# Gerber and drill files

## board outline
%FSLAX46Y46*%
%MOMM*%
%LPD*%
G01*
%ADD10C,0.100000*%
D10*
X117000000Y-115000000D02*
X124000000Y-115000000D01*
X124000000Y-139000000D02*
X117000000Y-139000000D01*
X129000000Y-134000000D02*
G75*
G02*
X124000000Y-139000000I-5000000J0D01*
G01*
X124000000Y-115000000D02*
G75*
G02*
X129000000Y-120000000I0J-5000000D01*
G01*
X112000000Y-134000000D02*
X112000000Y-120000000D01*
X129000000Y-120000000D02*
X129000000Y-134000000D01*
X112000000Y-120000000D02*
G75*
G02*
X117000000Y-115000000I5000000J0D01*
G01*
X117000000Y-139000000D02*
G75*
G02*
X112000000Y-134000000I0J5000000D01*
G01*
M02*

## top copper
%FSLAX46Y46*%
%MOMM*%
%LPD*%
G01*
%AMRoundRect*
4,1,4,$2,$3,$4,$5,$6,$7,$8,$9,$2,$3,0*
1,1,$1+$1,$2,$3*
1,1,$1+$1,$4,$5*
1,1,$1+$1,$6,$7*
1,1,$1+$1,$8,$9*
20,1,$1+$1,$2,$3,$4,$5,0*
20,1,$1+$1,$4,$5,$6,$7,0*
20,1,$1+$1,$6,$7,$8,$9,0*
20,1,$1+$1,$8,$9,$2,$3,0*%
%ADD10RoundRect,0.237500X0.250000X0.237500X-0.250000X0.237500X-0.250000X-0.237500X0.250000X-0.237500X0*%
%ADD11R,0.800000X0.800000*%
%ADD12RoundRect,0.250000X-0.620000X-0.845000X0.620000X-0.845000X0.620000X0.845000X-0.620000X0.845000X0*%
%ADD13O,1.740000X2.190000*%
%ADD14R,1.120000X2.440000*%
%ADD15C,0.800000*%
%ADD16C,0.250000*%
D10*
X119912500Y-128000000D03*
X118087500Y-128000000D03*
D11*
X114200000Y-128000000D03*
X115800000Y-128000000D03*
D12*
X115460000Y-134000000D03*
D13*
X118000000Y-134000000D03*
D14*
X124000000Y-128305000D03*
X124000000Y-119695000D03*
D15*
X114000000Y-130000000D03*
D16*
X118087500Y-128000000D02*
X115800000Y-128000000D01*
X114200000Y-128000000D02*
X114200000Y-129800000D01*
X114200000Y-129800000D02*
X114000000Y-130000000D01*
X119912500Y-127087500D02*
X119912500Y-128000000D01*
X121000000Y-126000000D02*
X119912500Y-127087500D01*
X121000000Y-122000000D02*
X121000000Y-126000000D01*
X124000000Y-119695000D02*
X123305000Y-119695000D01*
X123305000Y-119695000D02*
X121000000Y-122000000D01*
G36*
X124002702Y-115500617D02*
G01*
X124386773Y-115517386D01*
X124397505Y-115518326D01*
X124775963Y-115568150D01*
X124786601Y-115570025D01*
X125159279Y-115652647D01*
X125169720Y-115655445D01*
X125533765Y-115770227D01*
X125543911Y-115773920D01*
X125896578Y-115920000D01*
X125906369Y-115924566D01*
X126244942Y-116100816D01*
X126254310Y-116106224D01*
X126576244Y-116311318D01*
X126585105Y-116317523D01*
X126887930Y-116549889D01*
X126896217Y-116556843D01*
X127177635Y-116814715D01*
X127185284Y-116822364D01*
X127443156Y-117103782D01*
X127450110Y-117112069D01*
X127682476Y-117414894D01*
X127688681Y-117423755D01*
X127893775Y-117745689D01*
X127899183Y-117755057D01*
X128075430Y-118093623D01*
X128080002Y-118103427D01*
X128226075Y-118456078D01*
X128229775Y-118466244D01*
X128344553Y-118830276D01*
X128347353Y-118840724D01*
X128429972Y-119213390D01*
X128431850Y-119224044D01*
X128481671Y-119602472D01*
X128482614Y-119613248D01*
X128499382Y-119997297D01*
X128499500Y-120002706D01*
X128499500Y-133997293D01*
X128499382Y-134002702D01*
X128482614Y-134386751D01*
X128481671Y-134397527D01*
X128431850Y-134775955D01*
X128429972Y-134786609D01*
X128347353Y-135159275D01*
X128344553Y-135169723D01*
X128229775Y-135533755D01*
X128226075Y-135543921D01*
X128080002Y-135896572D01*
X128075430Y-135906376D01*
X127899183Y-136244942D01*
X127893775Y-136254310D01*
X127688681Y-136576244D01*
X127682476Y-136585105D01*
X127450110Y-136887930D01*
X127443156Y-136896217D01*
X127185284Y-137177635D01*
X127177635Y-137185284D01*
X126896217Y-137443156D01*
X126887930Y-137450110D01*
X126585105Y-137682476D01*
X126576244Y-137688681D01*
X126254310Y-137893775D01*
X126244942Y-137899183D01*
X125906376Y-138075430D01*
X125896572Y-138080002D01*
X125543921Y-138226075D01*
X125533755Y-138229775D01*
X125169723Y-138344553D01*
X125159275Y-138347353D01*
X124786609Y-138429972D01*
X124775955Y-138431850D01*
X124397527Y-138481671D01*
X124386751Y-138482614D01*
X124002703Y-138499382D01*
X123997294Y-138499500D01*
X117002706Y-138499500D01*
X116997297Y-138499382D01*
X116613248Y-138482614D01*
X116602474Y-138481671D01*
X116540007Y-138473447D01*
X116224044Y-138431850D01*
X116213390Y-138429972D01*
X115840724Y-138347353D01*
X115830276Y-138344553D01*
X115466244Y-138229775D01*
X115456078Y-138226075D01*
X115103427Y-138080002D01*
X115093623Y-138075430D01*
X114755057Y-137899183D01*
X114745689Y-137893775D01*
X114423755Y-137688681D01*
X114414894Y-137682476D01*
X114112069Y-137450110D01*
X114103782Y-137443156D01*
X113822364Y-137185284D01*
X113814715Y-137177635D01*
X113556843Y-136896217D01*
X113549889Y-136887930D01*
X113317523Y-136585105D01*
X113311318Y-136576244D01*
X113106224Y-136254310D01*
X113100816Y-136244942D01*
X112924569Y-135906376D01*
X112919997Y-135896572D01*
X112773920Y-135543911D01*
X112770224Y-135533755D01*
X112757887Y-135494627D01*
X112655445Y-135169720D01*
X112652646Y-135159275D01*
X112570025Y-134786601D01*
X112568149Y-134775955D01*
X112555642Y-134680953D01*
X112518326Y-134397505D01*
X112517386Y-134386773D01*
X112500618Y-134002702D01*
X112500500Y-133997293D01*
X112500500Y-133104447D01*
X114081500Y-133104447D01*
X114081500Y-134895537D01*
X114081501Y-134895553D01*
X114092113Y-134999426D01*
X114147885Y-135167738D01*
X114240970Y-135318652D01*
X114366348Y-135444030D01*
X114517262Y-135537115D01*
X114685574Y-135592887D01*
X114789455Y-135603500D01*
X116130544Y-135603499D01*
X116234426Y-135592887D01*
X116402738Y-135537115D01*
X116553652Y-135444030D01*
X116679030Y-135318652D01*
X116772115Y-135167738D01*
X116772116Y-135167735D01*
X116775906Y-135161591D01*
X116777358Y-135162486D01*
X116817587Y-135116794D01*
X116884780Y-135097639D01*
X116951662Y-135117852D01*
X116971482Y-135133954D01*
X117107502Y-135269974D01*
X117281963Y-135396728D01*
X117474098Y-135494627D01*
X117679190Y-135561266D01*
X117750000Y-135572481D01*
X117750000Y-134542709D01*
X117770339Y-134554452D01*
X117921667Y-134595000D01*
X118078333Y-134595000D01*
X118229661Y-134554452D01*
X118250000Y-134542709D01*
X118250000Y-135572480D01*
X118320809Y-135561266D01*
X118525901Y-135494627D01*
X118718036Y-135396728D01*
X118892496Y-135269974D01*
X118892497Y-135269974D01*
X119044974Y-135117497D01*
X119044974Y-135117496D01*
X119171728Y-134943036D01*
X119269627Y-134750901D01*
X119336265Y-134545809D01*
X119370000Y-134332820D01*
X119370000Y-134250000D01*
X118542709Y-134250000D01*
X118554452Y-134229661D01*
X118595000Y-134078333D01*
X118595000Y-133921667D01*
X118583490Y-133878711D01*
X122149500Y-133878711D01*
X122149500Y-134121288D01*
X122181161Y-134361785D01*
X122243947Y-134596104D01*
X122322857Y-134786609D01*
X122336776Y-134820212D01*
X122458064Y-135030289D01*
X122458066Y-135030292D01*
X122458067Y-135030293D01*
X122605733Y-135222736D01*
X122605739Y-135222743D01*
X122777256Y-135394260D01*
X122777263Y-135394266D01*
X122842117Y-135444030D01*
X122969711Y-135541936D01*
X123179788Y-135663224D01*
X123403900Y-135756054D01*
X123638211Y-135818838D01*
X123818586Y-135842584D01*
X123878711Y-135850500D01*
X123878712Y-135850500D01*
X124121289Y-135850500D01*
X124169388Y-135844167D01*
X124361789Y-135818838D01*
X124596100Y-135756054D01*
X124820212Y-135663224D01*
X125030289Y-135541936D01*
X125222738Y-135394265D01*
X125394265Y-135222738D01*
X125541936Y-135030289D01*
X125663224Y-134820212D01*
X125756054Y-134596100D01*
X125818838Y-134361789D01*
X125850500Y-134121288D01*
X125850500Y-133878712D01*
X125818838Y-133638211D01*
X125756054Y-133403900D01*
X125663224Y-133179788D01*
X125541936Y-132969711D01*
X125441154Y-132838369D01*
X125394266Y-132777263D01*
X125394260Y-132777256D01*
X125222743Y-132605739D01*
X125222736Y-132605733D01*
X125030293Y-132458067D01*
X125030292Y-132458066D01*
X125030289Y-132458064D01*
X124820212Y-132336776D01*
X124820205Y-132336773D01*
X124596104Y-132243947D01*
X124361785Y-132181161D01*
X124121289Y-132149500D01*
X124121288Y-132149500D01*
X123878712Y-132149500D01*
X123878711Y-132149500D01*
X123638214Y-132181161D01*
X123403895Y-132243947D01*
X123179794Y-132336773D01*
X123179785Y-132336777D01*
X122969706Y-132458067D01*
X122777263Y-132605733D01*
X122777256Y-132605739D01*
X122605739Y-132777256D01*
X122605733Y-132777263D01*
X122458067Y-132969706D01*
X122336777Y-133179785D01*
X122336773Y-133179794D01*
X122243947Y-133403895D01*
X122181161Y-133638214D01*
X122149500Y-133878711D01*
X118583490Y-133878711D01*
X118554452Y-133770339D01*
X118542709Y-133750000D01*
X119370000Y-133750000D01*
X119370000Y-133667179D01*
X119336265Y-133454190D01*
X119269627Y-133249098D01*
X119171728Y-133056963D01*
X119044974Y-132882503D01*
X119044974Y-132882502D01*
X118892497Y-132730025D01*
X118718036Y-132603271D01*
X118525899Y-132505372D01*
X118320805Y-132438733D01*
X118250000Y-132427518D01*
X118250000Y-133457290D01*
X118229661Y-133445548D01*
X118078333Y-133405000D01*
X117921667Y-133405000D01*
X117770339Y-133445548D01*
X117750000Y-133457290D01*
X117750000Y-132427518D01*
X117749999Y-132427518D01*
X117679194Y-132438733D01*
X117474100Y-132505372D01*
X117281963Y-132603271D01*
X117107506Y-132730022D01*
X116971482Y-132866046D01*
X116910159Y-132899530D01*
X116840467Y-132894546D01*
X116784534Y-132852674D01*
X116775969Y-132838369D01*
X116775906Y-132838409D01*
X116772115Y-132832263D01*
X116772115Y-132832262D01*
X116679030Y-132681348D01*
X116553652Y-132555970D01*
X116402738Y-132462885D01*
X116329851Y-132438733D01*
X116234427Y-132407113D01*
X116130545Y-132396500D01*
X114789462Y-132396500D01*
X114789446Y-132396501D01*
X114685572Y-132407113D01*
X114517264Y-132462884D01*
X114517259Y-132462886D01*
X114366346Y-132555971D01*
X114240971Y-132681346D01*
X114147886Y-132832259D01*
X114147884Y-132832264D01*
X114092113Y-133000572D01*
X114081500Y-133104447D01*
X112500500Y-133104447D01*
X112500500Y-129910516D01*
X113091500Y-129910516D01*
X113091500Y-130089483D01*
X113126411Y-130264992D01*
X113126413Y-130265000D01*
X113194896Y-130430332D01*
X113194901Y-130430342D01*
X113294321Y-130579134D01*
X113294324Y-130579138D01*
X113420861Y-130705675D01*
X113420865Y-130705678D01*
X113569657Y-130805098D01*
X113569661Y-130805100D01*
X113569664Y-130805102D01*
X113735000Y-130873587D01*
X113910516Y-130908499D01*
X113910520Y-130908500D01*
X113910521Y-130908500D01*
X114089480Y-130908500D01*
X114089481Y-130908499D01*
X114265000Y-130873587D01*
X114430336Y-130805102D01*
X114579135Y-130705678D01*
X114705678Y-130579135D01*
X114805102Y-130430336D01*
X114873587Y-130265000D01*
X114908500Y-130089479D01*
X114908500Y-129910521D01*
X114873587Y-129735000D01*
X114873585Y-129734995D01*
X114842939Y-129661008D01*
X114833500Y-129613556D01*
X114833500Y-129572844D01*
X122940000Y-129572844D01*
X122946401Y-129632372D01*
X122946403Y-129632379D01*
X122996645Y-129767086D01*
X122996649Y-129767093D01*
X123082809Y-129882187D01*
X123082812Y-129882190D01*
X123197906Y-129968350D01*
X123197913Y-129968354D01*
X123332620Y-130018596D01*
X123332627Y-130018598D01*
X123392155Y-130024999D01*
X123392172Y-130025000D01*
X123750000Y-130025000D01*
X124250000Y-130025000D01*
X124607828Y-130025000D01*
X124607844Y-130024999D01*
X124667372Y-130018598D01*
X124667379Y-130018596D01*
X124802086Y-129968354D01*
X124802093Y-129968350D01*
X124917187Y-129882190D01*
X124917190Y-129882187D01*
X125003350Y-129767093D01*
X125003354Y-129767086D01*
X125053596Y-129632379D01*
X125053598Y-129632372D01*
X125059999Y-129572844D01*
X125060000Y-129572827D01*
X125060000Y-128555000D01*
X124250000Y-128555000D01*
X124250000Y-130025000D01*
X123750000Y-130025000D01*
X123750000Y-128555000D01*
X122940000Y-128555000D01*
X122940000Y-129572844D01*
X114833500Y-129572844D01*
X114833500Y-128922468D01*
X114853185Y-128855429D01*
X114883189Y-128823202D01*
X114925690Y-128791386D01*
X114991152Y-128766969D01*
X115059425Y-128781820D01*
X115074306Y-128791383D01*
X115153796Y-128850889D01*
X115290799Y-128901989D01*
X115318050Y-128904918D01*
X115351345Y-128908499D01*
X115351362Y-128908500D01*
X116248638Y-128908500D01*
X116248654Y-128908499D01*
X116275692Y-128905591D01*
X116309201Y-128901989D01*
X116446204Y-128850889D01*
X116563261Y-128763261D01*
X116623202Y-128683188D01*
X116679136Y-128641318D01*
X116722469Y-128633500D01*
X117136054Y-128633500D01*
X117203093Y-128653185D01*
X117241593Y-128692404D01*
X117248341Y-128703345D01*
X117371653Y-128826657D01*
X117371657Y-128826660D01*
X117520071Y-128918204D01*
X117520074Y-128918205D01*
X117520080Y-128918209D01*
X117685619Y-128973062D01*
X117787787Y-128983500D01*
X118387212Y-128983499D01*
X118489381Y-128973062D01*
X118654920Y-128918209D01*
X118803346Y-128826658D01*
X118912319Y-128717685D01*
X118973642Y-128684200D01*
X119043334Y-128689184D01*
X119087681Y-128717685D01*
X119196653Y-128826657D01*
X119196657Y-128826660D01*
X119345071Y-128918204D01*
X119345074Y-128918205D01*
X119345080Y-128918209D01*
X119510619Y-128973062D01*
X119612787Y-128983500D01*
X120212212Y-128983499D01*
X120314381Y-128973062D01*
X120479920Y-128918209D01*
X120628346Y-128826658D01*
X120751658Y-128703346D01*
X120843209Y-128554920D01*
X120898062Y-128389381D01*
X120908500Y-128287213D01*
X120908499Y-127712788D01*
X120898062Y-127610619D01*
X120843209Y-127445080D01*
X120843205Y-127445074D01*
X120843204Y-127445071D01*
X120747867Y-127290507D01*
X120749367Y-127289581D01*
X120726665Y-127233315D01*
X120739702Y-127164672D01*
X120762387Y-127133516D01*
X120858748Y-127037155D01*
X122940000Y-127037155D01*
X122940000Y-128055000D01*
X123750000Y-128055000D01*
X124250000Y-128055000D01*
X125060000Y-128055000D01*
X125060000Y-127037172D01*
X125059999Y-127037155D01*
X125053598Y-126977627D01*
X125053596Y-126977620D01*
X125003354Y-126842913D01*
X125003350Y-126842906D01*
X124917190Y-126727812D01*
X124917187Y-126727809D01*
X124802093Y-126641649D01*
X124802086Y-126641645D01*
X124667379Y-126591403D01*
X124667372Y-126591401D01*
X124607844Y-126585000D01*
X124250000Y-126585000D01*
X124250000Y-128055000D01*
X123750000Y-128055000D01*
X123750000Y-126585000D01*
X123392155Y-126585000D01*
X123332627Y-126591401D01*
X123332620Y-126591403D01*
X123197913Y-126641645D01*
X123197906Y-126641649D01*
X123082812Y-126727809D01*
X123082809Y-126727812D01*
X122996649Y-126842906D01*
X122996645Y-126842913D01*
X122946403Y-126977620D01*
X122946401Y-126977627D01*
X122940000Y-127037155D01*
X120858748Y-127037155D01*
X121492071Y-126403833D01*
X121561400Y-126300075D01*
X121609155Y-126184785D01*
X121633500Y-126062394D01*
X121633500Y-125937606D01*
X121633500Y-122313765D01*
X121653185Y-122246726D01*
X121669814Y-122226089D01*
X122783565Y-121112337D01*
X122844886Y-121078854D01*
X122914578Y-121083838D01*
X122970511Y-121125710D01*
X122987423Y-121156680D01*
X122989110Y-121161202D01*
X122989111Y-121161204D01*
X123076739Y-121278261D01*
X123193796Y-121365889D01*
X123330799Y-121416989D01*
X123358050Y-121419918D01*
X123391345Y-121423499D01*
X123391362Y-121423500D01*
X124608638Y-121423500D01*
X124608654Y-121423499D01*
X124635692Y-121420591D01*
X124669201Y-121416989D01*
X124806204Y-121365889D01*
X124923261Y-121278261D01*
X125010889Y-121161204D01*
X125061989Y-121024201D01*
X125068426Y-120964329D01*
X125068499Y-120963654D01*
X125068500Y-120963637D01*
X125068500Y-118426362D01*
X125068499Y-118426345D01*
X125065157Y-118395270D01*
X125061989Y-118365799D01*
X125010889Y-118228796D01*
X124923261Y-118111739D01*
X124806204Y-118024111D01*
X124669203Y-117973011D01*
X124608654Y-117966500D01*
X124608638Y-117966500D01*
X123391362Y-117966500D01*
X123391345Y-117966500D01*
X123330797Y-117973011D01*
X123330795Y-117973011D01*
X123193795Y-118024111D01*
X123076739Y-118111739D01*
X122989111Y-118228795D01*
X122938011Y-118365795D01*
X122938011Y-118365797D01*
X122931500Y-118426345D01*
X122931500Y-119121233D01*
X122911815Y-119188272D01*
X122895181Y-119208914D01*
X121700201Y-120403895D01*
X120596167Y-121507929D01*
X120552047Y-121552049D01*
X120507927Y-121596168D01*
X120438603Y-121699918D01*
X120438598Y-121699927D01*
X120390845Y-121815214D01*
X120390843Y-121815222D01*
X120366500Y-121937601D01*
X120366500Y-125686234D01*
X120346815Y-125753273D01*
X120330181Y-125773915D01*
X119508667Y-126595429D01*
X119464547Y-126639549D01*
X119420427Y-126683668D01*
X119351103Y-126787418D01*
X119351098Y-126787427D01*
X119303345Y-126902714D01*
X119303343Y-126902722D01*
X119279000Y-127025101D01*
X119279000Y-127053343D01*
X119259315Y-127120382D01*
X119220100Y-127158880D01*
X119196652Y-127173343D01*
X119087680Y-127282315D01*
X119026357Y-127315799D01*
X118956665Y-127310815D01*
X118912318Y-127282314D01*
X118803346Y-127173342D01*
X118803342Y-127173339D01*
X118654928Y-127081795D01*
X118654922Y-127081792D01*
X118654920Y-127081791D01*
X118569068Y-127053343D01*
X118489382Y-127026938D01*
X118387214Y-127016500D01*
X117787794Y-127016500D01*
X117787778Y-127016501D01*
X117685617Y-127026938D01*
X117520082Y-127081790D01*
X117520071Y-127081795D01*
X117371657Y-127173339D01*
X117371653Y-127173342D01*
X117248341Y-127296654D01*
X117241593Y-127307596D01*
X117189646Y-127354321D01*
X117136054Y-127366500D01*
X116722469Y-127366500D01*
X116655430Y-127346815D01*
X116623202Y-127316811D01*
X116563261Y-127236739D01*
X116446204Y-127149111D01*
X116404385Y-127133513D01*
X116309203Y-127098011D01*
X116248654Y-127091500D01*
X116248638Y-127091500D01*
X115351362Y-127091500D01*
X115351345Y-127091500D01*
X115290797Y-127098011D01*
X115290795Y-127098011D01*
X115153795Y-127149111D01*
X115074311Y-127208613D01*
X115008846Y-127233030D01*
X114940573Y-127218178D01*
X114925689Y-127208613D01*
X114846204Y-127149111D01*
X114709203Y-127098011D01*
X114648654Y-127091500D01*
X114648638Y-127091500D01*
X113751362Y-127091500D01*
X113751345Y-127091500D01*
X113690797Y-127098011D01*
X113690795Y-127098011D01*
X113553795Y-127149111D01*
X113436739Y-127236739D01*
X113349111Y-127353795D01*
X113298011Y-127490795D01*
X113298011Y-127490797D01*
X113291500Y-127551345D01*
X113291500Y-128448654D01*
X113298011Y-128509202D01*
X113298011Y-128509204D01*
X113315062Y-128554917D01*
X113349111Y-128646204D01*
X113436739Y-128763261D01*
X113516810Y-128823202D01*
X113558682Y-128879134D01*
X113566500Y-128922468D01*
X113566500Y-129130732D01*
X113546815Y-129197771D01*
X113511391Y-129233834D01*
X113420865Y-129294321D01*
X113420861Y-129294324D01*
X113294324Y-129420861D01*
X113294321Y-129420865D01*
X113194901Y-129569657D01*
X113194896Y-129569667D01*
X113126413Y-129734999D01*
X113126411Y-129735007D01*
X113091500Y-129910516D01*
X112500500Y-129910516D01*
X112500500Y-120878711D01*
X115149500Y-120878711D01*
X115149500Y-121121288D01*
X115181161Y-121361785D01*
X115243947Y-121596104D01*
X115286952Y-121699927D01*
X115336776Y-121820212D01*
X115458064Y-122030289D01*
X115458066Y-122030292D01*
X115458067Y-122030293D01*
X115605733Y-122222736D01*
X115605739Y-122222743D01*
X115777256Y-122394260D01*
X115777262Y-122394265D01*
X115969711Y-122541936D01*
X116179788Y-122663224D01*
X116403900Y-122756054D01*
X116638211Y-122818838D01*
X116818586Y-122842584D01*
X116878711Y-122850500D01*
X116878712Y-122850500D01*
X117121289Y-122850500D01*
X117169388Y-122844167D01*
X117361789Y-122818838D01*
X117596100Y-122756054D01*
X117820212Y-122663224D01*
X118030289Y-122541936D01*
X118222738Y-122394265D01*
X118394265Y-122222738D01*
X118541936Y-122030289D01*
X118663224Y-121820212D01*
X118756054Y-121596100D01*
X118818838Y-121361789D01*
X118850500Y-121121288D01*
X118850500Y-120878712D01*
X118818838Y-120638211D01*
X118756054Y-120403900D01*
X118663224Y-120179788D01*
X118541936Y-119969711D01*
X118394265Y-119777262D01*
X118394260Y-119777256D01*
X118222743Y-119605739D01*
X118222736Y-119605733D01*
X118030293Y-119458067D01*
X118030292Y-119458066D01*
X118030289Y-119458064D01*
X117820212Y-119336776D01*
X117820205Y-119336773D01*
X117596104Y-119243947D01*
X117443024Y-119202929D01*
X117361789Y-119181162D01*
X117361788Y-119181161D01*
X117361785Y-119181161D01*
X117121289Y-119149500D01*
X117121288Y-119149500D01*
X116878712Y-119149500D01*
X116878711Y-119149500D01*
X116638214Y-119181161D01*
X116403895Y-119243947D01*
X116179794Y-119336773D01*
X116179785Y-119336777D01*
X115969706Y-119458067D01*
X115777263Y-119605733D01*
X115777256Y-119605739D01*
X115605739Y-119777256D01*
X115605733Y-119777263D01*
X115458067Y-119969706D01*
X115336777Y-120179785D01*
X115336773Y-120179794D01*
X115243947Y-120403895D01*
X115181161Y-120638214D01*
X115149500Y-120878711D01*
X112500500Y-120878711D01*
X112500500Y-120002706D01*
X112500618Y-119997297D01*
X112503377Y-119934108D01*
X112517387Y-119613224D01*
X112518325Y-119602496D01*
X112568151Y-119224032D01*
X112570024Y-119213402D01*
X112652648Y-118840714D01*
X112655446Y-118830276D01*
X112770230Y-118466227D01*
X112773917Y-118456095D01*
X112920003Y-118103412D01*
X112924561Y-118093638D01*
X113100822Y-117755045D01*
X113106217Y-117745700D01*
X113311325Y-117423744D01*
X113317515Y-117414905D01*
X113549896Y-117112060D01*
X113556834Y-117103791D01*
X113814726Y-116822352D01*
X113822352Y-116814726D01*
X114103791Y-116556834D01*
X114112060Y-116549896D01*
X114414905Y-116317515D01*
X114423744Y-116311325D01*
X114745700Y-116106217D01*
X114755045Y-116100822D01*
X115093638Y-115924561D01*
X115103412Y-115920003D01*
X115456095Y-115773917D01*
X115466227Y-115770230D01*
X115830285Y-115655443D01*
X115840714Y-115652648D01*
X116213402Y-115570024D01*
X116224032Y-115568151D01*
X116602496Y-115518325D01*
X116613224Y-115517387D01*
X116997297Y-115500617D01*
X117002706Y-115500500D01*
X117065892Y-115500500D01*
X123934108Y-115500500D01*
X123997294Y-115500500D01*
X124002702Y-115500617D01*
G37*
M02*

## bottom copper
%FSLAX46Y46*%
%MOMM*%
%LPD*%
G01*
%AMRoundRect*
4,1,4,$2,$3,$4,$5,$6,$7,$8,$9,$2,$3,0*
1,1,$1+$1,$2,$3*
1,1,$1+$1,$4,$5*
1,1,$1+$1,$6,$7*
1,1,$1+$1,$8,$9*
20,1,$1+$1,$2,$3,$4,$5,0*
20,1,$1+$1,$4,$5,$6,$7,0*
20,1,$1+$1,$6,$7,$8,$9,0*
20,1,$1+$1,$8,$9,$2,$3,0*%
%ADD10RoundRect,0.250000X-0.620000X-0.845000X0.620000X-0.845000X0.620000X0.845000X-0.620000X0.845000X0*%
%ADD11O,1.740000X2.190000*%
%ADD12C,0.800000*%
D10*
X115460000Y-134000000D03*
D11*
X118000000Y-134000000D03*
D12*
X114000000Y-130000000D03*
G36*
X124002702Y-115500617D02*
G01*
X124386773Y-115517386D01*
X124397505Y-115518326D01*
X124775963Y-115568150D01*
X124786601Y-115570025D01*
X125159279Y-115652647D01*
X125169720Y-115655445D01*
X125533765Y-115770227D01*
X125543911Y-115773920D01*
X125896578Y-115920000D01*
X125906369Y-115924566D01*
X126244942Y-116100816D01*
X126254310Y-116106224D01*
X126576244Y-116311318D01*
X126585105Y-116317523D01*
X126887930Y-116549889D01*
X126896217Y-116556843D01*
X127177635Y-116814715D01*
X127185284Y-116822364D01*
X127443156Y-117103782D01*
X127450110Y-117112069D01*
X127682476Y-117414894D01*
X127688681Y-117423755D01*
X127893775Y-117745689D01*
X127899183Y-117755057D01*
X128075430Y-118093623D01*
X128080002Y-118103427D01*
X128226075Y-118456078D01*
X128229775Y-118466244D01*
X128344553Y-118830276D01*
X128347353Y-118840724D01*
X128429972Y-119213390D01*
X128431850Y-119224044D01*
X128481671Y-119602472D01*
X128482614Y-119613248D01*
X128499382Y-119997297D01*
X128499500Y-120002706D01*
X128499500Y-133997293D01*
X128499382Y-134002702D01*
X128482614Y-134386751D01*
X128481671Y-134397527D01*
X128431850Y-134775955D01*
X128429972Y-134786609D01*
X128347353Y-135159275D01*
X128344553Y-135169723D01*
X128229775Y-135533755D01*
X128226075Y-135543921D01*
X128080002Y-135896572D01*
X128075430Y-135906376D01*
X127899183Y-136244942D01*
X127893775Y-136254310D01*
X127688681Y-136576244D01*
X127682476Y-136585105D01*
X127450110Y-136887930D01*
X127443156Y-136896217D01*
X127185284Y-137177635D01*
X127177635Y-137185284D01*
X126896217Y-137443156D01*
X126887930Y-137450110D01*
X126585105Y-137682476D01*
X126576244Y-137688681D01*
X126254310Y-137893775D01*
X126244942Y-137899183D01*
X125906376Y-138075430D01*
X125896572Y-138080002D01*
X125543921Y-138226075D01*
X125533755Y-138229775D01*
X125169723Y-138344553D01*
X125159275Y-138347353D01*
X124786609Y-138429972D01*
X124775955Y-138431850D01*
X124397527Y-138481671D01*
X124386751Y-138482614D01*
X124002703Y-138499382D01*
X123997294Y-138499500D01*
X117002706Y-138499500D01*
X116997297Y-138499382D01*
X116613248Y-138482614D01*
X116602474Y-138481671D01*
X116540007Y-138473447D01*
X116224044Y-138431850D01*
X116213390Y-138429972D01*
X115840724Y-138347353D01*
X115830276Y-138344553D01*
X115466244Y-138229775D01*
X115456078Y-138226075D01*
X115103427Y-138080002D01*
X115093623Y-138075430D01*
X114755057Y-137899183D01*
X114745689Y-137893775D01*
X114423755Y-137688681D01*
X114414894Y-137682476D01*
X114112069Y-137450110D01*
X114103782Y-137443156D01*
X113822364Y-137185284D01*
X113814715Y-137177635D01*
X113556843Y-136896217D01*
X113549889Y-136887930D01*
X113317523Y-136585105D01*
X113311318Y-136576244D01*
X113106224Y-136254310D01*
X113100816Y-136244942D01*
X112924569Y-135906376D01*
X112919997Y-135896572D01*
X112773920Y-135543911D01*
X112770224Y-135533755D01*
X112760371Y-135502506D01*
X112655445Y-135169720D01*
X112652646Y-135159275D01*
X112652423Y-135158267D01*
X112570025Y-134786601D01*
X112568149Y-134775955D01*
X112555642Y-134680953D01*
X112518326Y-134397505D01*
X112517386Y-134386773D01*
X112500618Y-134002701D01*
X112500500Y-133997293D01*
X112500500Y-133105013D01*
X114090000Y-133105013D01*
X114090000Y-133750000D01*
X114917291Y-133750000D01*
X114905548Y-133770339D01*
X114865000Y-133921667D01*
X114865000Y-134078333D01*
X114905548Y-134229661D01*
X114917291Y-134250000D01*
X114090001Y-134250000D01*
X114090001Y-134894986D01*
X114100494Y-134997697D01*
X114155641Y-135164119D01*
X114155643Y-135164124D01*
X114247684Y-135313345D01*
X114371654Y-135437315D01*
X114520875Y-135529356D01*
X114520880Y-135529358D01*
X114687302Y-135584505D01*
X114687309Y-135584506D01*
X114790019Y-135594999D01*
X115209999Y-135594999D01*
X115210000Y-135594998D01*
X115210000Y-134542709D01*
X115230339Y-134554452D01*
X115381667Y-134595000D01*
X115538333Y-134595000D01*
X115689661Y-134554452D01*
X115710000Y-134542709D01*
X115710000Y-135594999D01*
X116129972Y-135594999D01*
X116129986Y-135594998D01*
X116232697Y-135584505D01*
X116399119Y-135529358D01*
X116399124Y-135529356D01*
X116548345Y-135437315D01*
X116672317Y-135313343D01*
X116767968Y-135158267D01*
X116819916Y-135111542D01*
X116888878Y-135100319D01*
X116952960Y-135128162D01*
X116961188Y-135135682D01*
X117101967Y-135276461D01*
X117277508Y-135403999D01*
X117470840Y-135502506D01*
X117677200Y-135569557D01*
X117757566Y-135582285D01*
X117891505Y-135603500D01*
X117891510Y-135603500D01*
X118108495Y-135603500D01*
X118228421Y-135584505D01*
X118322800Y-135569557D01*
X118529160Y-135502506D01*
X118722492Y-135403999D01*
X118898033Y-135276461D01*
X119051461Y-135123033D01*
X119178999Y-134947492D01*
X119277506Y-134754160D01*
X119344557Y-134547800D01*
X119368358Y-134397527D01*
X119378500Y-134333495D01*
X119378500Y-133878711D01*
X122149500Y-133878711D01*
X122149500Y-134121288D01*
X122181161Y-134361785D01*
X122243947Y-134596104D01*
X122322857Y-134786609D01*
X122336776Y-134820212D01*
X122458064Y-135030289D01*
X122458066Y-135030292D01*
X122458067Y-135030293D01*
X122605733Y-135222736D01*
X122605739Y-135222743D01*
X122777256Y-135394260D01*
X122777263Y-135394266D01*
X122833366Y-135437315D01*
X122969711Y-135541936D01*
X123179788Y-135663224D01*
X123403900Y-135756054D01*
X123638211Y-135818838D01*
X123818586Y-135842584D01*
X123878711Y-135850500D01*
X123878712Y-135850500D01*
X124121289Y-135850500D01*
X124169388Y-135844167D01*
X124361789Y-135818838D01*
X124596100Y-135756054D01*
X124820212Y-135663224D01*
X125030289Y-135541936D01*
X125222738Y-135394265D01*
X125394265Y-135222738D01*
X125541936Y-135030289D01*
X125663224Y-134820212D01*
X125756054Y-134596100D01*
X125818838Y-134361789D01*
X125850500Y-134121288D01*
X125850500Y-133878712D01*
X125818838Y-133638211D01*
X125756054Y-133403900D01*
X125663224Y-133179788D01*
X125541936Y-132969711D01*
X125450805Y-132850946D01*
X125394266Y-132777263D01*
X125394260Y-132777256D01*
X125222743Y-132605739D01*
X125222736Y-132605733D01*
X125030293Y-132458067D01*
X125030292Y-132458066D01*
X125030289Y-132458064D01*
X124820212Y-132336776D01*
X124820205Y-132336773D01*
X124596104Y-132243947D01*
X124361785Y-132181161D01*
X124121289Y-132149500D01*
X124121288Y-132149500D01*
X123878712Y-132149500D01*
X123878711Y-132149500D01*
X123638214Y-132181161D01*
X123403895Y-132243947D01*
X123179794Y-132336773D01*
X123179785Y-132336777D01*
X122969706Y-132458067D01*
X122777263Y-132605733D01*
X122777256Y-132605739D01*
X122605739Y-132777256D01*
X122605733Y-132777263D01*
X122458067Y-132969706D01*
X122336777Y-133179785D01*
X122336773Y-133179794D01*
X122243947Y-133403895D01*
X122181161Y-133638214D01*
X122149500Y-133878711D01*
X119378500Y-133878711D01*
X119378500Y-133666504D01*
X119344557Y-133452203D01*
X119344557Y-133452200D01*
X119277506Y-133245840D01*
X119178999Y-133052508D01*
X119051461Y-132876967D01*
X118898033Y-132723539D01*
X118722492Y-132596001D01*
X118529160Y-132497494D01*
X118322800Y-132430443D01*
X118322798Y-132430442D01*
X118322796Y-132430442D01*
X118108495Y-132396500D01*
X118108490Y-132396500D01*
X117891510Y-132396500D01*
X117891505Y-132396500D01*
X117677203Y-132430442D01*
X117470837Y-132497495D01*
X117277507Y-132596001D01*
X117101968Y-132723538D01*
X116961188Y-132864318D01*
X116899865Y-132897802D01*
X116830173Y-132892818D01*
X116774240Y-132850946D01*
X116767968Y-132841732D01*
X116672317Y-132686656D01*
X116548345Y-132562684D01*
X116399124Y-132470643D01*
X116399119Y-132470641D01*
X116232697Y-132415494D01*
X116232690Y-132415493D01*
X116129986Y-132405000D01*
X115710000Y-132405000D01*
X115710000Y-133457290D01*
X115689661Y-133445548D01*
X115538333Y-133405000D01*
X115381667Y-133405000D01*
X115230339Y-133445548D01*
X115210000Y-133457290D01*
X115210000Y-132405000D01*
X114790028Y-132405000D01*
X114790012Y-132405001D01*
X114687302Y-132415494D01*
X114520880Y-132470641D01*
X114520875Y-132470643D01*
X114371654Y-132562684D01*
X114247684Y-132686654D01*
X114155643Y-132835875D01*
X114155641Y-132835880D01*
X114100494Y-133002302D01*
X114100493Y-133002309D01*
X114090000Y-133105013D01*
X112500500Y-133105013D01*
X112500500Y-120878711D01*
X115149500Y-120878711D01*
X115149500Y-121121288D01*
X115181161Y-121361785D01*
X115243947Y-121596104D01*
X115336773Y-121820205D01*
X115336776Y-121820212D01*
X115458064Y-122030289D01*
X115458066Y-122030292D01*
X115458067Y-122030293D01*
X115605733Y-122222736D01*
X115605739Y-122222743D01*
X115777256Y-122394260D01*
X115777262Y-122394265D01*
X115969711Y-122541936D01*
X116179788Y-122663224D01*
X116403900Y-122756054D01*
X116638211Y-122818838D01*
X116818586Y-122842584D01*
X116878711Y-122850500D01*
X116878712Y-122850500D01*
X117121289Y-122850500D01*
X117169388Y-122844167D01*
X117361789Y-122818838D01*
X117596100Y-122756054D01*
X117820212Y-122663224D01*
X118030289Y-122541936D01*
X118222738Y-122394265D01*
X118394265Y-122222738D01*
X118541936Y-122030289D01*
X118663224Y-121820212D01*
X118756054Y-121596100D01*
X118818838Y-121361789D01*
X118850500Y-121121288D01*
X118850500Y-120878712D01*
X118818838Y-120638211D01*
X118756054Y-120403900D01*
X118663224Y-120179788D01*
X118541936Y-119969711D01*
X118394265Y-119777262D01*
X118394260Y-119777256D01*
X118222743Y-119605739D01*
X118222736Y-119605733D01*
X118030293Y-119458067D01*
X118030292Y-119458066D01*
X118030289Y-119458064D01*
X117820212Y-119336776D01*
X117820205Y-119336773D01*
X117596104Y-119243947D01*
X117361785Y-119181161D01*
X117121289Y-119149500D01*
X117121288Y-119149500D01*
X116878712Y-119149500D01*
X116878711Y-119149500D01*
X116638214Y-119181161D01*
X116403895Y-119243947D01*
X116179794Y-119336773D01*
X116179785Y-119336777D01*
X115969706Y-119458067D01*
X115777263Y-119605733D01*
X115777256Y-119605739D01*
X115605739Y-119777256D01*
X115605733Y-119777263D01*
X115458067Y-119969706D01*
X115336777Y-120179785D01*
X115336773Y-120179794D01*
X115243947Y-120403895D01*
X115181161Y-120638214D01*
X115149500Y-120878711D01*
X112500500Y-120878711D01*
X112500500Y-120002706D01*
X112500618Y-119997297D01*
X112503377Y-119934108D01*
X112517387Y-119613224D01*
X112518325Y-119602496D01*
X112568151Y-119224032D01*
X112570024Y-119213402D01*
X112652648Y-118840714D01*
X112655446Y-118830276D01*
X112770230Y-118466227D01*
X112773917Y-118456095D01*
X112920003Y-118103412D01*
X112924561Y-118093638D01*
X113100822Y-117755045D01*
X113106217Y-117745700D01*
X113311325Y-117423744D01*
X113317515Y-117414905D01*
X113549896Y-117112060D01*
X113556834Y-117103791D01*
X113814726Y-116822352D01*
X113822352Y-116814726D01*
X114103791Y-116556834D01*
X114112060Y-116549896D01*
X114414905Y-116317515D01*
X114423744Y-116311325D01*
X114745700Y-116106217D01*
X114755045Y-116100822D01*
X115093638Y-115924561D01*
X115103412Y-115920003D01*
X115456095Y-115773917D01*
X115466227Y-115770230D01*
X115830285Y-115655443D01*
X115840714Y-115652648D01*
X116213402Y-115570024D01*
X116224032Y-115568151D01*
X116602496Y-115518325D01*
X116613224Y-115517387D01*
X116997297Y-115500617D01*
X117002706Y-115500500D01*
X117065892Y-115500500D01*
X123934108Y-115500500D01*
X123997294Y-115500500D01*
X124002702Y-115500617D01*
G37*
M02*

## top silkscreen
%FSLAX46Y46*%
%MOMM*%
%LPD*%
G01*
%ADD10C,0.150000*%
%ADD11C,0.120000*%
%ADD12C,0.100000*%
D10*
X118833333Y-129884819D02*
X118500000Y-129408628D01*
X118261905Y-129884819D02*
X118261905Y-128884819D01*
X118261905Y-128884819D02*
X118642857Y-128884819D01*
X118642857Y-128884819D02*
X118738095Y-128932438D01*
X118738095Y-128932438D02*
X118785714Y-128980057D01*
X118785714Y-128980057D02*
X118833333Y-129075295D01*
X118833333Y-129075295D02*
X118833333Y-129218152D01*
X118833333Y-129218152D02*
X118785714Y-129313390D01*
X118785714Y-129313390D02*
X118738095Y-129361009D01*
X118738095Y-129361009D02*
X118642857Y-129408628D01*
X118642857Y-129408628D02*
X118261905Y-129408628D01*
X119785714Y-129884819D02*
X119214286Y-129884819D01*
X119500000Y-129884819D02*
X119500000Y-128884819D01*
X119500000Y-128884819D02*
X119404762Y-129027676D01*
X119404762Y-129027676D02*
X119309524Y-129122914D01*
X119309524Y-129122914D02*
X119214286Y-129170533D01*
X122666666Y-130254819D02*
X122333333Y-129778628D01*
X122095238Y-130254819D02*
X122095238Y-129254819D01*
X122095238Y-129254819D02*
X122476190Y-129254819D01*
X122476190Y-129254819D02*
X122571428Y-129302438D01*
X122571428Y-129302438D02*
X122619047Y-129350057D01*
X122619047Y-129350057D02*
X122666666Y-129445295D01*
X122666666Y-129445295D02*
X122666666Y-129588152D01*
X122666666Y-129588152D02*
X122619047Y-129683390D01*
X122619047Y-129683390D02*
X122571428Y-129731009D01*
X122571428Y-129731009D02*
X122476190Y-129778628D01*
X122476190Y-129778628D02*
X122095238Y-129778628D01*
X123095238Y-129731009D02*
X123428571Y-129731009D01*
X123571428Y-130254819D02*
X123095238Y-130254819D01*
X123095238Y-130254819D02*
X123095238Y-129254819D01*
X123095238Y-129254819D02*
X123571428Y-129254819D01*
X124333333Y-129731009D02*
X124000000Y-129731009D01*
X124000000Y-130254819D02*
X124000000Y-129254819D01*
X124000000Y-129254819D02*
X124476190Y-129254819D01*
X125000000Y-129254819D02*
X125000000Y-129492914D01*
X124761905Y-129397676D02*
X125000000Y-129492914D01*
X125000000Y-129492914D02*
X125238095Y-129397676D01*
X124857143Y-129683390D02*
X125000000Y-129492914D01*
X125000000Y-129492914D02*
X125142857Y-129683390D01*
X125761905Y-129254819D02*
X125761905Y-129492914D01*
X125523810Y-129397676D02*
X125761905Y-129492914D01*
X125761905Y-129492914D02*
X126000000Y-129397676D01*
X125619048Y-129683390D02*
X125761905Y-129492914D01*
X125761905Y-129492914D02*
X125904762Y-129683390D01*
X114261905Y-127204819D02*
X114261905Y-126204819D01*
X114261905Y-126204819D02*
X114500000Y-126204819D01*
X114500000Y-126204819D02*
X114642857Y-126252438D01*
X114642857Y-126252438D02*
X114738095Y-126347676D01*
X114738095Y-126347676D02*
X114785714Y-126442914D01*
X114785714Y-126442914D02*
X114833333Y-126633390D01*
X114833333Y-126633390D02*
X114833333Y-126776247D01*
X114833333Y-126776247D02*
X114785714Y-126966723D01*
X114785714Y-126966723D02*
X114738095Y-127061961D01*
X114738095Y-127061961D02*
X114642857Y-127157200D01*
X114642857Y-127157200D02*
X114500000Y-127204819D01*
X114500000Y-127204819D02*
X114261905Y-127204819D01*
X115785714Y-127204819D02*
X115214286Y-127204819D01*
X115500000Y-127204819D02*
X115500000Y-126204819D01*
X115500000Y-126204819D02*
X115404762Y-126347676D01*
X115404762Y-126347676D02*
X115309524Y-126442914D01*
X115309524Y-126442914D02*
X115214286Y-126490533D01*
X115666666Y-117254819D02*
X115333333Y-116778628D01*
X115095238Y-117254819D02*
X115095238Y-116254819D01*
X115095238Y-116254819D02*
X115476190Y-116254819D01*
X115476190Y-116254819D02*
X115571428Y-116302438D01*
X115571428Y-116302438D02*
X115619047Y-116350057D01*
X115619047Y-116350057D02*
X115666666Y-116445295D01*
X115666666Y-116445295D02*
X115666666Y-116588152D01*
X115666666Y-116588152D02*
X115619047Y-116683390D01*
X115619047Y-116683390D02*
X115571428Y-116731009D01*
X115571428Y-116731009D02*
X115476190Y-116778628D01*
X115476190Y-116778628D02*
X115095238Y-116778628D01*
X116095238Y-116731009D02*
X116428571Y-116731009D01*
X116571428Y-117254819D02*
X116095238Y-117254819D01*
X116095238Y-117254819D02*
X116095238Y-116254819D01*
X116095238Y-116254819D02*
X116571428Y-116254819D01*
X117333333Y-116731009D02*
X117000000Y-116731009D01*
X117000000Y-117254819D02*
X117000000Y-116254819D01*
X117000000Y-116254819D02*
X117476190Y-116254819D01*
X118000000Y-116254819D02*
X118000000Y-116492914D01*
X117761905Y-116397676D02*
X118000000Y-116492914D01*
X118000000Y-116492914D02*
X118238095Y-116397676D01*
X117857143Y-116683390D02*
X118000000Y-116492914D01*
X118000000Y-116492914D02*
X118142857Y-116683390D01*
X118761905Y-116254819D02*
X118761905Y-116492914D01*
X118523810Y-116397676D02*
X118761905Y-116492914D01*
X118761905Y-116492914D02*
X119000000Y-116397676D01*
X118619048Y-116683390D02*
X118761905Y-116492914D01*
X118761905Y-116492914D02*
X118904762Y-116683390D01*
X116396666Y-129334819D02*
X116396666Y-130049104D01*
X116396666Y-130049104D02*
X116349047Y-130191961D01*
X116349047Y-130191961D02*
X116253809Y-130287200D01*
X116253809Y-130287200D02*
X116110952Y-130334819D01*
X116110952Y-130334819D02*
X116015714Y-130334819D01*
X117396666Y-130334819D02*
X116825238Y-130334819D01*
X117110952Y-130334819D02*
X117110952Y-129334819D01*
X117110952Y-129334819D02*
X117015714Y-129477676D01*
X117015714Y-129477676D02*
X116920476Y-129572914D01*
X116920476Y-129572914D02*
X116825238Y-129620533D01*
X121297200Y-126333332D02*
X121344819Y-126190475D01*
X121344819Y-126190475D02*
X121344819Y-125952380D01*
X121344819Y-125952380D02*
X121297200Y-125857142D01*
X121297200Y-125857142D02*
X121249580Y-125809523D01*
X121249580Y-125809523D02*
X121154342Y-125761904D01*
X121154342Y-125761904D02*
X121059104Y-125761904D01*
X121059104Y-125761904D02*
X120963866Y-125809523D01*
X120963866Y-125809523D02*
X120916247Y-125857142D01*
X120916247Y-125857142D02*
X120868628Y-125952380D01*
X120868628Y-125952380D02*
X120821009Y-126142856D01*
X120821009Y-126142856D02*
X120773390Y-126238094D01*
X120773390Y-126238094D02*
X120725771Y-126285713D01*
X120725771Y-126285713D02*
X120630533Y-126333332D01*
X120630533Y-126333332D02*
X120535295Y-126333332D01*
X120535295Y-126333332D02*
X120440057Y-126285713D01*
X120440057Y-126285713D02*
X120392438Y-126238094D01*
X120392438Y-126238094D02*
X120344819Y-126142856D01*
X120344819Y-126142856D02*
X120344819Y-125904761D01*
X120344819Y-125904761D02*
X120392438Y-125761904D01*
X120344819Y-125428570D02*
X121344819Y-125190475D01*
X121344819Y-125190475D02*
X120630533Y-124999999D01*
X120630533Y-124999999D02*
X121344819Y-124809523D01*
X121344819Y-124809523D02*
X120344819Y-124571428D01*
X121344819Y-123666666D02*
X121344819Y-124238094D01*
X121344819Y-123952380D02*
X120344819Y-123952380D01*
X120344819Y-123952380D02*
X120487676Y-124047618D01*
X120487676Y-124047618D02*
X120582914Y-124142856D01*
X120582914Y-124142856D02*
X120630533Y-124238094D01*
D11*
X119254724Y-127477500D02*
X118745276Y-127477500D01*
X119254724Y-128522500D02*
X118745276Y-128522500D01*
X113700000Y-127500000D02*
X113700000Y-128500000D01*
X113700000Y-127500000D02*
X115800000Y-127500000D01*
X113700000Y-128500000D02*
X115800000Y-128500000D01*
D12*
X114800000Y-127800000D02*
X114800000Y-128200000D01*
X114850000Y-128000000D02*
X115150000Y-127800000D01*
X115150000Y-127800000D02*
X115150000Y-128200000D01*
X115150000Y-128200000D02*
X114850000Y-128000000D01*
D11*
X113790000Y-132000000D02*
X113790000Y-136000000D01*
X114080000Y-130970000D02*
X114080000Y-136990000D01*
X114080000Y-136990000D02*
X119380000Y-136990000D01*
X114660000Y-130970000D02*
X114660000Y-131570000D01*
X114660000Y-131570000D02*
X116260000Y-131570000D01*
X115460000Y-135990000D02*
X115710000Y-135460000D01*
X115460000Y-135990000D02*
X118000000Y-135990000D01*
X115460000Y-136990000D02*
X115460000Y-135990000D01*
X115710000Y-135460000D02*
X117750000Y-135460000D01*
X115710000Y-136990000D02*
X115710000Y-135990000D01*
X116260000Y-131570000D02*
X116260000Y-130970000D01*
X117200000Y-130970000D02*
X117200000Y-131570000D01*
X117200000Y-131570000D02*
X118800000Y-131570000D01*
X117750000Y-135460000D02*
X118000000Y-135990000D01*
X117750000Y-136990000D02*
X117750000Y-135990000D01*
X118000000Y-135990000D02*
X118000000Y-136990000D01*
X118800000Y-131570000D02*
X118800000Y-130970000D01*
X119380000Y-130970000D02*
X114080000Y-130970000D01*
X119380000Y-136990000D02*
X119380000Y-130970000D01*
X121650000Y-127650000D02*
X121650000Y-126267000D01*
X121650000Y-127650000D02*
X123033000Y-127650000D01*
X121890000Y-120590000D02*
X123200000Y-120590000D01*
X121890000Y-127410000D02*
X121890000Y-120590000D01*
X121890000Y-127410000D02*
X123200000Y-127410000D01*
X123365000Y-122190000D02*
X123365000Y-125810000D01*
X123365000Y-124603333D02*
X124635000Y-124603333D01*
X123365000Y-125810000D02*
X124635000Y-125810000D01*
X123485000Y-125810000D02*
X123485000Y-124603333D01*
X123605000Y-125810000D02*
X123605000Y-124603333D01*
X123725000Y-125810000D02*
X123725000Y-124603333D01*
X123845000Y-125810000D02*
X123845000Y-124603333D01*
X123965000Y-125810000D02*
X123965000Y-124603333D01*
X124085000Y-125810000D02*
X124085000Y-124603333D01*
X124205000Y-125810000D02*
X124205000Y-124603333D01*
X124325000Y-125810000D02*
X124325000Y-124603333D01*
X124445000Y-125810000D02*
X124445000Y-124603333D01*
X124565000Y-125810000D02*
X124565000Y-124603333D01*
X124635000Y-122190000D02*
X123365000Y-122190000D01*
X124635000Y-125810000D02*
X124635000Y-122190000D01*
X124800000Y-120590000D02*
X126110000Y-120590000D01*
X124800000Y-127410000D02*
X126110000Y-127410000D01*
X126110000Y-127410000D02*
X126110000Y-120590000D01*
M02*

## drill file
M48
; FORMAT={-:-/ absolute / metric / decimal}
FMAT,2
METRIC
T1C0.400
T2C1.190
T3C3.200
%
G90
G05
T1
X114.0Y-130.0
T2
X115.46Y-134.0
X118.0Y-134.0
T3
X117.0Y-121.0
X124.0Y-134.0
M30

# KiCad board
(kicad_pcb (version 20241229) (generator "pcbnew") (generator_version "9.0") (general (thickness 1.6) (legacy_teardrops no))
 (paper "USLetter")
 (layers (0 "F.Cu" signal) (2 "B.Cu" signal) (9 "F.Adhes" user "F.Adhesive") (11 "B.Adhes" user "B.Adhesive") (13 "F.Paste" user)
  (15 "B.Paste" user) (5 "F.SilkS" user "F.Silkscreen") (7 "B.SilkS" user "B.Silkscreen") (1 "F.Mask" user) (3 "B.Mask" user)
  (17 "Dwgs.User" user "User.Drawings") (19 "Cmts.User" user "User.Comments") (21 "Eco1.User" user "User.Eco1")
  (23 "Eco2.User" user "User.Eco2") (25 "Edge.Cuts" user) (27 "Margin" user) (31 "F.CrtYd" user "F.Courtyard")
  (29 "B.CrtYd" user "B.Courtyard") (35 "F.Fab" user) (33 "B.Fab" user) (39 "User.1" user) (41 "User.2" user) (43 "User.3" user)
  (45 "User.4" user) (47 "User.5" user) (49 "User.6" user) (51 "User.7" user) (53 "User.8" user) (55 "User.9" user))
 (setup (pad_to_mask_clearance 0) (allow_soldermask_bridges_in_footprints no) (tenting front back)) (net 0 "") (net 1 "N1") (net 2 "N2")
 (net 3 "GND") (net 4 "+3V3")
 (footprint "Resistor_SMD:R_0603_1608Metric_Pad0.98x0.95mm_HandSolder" (layer "F.Cu") (at 119 128 180)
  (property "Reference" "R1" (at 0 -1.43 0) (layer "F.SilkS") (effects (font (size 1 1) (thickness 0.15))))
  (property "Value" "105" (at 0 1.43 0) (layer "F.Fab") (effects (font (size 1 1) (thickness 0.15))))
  (fp_line (start -0.254724 0.5225) (end 0.254724 0.5225) (stroke (width 0.12) (type solid)) (layer "F.SilkS"))
  (fp_line (start -0.254724 -0.5225) (end 0.254724 -0.5225) (stroke (width 0.12) (type solid)) (layer "F.SilkS"))
  (pad "1" smd roundrect (at -0.9125 0 180) (size 0.975 0.95) (layers "F.Cu" "F.Mask" "F.Paste") (roundrect_rratio 0.25) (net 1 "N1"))
  (pad "2" smd roundrect (at 0.9125 0 180) (size 0.975 0.95) (layers "F.Cu" "F.Mask" "F.Paste") (roundrect_rratio 0.25) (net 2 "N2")))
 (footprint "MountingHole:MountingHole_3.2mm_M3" (layer "F.Cu") (at 124 134)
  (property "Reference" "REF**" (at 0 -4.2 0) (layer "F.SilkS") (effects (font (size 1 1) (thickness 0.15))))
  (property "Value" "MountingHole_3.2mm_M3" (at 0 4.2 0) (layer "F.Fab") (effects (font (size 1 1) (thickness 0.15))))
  (pad "" np_thru_hole circle (at 0 0) (size 3.2 3.2) (drill 3.2) (layers "*.Cu" "*.Mask")))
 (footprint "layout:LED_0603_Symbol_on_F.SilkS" (layer "F.Cu") (at 115 128)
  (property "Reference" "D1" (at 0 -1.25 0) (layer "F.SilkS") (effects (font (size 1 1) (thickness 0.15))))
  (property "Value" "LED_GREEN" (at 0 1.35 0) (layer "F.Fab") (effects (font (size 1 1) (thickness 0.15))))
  (fp_line (start -1.3 -0.5) (end -1.3 0.5) (stroke (width 0.12) (type solid)) (layer "F.SilkS"))
  (fp_line (start -1.3 -0.5) (end 0.8 -0.5) (stroke (width 0.12) (type solid)) (layer "F.SilkS"))
  (fp_line (start -1.3 0.5) (end 0.8 0.5) (stroke (width 0.12) (type solid)) (layer "F.SilkS"))
  (fp_line (start -0.2 -0.2) (end -0.2 0.2) (stroke (width 0.1) (type solid)) (layer "F.SilkS"))
  (fp_line (start -0.15 0) (end 0.15 -0.2) (stroke (width 0.1) (type solid)) (layer "F.SilkS"))
  (fp_line (start 0.15 -0.2) (end 0.15 0.2) (stroke (width 0.1) (type solid)) (layer "F.SilkS"))
  (fp_line (start 0.15 0.2) (end -0.15 0) (stroke (width 0.1) (type solid)) (layer "F.SilkS"))
  (pad "1" smd rect (at -0.8 0 180) (size 0.8 0.8) (layers "F.Cu" "F.Mask" "F.Paste") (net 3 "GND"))
  (pad "2" smd rect (at 0.8 0 180) (size 0.8 0.8) (layers "F.Cu" "F.Mask" "F.Paste") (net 2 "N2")))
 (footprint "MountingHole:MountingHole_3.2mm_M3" (layer "F.Cu") (at 117 121)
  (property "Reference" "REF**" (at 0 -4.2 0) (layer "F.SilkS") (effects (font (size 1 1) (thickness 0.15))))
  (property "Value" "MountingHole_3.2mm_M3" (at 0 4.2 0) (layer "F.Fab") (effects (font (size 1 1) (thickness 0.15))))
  (pad "" np_thru_hole circle (at 0 0) (size 3.2 3.2) (drill 3.2) (layers "*.Cu" "*.Mask")))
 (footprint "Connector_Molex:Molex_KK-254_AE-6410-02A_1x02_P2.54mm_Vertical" (layer "F.Cu") (at 115.46 134)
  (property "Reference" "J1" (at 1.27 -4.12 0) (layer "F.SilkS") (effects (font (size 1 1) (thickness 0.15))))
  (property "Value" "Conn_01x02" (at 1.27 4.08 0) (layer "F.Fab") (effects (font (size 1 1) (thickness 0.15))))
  (fp_line (start -1.67 -2) (end -1.67 2) (stroke (width 0.12) (type solid)) (layer "F.SilkS"))
  (fp_line (start -1.38 -3.03) (end -1.38 2.99) (stroke (width 0.12) (type solid)) (layer "F.SilkS"))
  (fp_line (start -1.38 2.99) (end 3.92 2.99) (stroke (width 0.12) (type solid)) (layer "F.SilkS"))
  (fp_line (start -0.8 -3.03) (end -0.8 -2.43) (stroke (width 0.12) (type solid)) (layer "F.SilkS"))
  (fp_line (start -0.8 -2.43) (end 0.8 -2.43) (stroke (width 0.12) (type solid)) (layer "F.SilkS"))
  (fp_line (start 0 1.99) (end 0.25 1.46) (stroke (width 0.12) (type solid)) (layer "F.SilkS"))
  (fp_line (start 0 1.99) (end 2.54 1.99) (stroke (width 0.12) (type solid)) (layer "F.SilkS"))
  (fp_line (start 0 2.99) (end 0 1.99) (stroke (width 0.12) (type solid)) (layer "F.SilkS"))
  (fp_line (start 0.25 1.46) (end 2.29 1.46) (stroke (width 0.12) (type solid)) (layer "F.SilkS"))
  (fp_line (start 0.25 2.99) (end 0.25 1.99) (stroke (width 0.12) (type solid)) (layer "F.SilkS"))
  (fp_line (start 0.8 -2.43) (end 0.8 -3.03) (stroke (width 0.12) (type solid)) (layer "F.SilkS"))
  (fp_line (start 1.74 -3.03) (end 1.74 -2.43) (stroke (width 0.12) (type solid)) (layer "F.SilkS"))
  (fp_line (start 1.74 -2.43) (end 3.34 -2.43) (stroke (width 0.12) (type solid)) (layer "F.SilkS"))
  (fp_line (start 2.29 1.46) (end 2.54 1.99) (stroke (width 0.12) (type solid)) (layer "F.SilkS"))
  (fp_line (start 2.29 2.99) (end 2.29 1.99) (stroke (width 0.12) (type solid)) (layer "F.SilkS"))
  (fp_line (start 2.54 1.99) (end 2.54 2.99) (stroke (width 0.12) (type solid)) (layer "F.SilkS"))
  (fp_line (start 3.34 -2.43) (end 3.34 -3.03) (stroke (width 0.12) (type solid)) (layer "F.SilkS"))
  (fp_line (start 3.92 -3.03) (end -1.38 -3.03) (stroke (width 0.12) (type solid)) (layer "F.SilkS"))
  (fp_line (start 3.92 2.99) (end 3.92 -3.03) (stroke (width 0.12) (type solid)) (layer "F.SilkS"))
  (pad "1" thru_hole roundrect (at 0 0) (size 1.74 2.19) (drill 1.19) (layers "*.Cu" "*.Mask") (remove_unused_layers no)
   (roundrect_rratio 0.143678) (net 3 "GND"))
  (pad "2" thru_hole oval (at 2.54 0) (size 1.74 2.19) (drill 1.19) (layers "*.Cu" "*.Mask") (remove_unused_layers no) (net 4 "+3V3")))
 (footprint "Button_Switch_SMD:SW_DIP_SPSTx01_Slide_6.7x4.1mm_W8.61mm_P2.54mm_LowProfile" (layer "F.Cu") (at 124 124 90)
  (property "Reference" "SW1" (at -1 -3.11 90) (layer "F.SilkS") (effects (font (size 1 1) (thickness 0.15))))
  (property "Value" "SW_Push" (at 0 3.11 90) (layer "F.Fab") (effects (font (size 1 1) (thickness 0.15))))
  (fp_line (start -3.65 -2.35) (end -2.267 -2.35) (stroke (width 0.12) (type solid)) (layer "F.SilkS"))
  (fp_line (start -3.65 -2.35) (end -3.65 -0.967) (stroke (width 0.12) (type solid)) (layer "F.SilkS"))
  (fp_line (start 3.41 -2.11) (end 3.41 -0.8) (stroke (width 0.12) (type solid)) (layer "F.SilkS"))
  (fp_line (start -3.41 -2.11) (end 3.41 -2.11) (stroke (width 0.12) (type solid)) (layer "F.SilkS"))
  (fp_line (start -3.41 -2.11) (end -3.41 -0.8) (stroke (width 0.12) (type solid)) (layer "F.SilkS"))
  (fp_line (start 1.81 -0.635) (end -1.81 -0.635) (stroke (width 0.12) (type solid)) (layer "F.SilkS"))
  (fp_line (start -0.603333 -0.635) (end -0.603333 0.635) (stroke (width 0.12) (type solid)) (layer "F.SilkS"))
  (fp_line (start -1.81 -0.635) (end -1.81 0.635) (stroke (width 0.12) (type solid)) (layer "F.SilkS"))
  (fp_line (start -1.81 -0.515) (end -0.603333 -0.515) (stroke (width 0.12) (type solid)) (layer "F.SilkS"))
  (fp_line (start -1.81 -0.395) (end -0.603333 -0.395) (stroke (width 0.12) (type solid)) (layer "F.SilkS"))
  (fp_line (start -1.81 -0.275) (end -0.603333 -0.275) (stroke (width 0.12) (type solid)) (layer "F.SilkS"))
  (fp_line (start -1.81 -0.155) (end -0.603333 -0.155) (stroke (width 0.12) (type solid)) (layer "F.SilkS"))
  (fp_line (start -1.81 -0.035) (end -0.603333 -0.035) (stroke (width 0.12) (type solid)) (layer "F.SilkS"))
  (fp_line (start -1.81 0.085) (end -0.603333 0.085) (stroke (width 0.12) (type solid)) (layer "F.SilkS"))
  (fp_line (start -1.81 0.205) (end -0.603333 0.205) (stroke (width 0.12) (type solid)) (layer "F.SilkS"))
  (fp_line (start -1.81 0.325) (end -0.603333 0.325) (stroke (width 0.12) (type solid)) (layer "F.SilkS"))
  (fp_line (start -1.81 0.445) (end -0.603333 0.445) (stroke (width 0.12) (type solid)) (layer "F.SilkS"))
  (fp_line (start -1.81 0.565) (end -0.603333 0.565) (stroke (width 0.12) (type solid)) (layer "F.SilkS"))
  (fp_line (start 1.81 0.635) (end 1.81 -0.635) (stroke (width 0.12) (type solid)) (layer "F.SilkS"))
  (fp_line (start -1.81 0.635) (end 1.81 0.635) (stroke (width 0.12) (type solid)) (layer "F.SilkS"))
  (fp_line (start 3.41 0.8) (end 3.41 2.11) (stroke (width 0.12) (type solid)) (layer "F.SilkS"))
  (fp_line (start -3.41 0.8) (end -3.41 2.11) (stroke (width 0.12) (type solid)) (layer "F.SilkS"))
  (fp_line (start -3.41 2.11) (end 3.41 2.11) (stroke (width 0.12) (type solid)) (layer "F.SilkS"))
  (pad "1" smd rect (at -4.305 0 90) (size 2.44 1.12) (layers "F.Cu" "F.Mask" "F.Paste") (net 4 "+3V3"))
  (pad "2" smd rect (at 4.305 0 90) (size 2.44 1.12) (layers "F.Cu" "F.Mask" "F.Paste") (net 1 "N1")))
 (gr_line (start 117 115) (end 124 115) (stroke (width 0.1) (type default)) (layer "Edge.Cuts"))
 (gr_line (start 124 139) (end 117 139) (stroke (width 0.1) (type default)) (layer "Edge.Cuts"))
 (gr_arc (start 129 134) (mid 127.535534 137.535534) (end 124 139) (stroke (width 0.1) (type default)) (layer "Edge.Cuts"))
 (gr_arc (start 124 115) (mid 127.535534 116.464466) (end 129 120) (stroke (width 0.1) (type default)) (layer "Edge.Cuts"))
 (gr_line (start 112 134) (end 112 120) (stroke (width 0.1) (type default)) (layer "Edge.Cuts"))
 (gr_line (start 129 120) (end 129 134) (stroke (width 0.1) (type default)) (layer "Edge.Cuts"))
 (gr_arc (start 112 120) (mid 113.464466 116.464466) (end 117 115) (stroke (width 0.1) (type default)) (layer "Edge.Cuts"))
 (gr_arc (start 117 139) (mid 113.464466 137.535534) (end 112 134) (stroke (width 0.1) (type default)) (layer "Edge.Cuts"))
 (segment (start 118.0875 128) (end 115.8 128) (width 0.25) (layer "F.Cu") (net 2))
 (segment (start 114.2 128) (end 114.2 129.8) (width 0.25) (layer "F.Cu") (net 3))
 (segment (start 114.2 129.8) (end 114 130) (width 0.25) (layer "F.Cu") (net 3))
 (via (at 114 130) (size 0.8) (drill 0.4) (layers "F.Cu" "B.Cu") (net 3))
 (segment (start 119.9125 127.0875) (end 119.9125 128) (width 0.25) (layer "F.Cu") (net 1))
 (segment (start 121 126) (end 119.9125 127.0875) (width 0.25) (layer "F.Cu") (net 1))
 (segment (start 121 122) (end 121 126) (width 0.25) (layer "F.Cu") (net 1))
 (segment (start 124 119.695) (end 123.305 119.695) (width 0.25) (layer "F.Cu") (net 1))
 (segment (start 123.305 119.695) (end 121 122) (width 0.25) (layer "F.Cu") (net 1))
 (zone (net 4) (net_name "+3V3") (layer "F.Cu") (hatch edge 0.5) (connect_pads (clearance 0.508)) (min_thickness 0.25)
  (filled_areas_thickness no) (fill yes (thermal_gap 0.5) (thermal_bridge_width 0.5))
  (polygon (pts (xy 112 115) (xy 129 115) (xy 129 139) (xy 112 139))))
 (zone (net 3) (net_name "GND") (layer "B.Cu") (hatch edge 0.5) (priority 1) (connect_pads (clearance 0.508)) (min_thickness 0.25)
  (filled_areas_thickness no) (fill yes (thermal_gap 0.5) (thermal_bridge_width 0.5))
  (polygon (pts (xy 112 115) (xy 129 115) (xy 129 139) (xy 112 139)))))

